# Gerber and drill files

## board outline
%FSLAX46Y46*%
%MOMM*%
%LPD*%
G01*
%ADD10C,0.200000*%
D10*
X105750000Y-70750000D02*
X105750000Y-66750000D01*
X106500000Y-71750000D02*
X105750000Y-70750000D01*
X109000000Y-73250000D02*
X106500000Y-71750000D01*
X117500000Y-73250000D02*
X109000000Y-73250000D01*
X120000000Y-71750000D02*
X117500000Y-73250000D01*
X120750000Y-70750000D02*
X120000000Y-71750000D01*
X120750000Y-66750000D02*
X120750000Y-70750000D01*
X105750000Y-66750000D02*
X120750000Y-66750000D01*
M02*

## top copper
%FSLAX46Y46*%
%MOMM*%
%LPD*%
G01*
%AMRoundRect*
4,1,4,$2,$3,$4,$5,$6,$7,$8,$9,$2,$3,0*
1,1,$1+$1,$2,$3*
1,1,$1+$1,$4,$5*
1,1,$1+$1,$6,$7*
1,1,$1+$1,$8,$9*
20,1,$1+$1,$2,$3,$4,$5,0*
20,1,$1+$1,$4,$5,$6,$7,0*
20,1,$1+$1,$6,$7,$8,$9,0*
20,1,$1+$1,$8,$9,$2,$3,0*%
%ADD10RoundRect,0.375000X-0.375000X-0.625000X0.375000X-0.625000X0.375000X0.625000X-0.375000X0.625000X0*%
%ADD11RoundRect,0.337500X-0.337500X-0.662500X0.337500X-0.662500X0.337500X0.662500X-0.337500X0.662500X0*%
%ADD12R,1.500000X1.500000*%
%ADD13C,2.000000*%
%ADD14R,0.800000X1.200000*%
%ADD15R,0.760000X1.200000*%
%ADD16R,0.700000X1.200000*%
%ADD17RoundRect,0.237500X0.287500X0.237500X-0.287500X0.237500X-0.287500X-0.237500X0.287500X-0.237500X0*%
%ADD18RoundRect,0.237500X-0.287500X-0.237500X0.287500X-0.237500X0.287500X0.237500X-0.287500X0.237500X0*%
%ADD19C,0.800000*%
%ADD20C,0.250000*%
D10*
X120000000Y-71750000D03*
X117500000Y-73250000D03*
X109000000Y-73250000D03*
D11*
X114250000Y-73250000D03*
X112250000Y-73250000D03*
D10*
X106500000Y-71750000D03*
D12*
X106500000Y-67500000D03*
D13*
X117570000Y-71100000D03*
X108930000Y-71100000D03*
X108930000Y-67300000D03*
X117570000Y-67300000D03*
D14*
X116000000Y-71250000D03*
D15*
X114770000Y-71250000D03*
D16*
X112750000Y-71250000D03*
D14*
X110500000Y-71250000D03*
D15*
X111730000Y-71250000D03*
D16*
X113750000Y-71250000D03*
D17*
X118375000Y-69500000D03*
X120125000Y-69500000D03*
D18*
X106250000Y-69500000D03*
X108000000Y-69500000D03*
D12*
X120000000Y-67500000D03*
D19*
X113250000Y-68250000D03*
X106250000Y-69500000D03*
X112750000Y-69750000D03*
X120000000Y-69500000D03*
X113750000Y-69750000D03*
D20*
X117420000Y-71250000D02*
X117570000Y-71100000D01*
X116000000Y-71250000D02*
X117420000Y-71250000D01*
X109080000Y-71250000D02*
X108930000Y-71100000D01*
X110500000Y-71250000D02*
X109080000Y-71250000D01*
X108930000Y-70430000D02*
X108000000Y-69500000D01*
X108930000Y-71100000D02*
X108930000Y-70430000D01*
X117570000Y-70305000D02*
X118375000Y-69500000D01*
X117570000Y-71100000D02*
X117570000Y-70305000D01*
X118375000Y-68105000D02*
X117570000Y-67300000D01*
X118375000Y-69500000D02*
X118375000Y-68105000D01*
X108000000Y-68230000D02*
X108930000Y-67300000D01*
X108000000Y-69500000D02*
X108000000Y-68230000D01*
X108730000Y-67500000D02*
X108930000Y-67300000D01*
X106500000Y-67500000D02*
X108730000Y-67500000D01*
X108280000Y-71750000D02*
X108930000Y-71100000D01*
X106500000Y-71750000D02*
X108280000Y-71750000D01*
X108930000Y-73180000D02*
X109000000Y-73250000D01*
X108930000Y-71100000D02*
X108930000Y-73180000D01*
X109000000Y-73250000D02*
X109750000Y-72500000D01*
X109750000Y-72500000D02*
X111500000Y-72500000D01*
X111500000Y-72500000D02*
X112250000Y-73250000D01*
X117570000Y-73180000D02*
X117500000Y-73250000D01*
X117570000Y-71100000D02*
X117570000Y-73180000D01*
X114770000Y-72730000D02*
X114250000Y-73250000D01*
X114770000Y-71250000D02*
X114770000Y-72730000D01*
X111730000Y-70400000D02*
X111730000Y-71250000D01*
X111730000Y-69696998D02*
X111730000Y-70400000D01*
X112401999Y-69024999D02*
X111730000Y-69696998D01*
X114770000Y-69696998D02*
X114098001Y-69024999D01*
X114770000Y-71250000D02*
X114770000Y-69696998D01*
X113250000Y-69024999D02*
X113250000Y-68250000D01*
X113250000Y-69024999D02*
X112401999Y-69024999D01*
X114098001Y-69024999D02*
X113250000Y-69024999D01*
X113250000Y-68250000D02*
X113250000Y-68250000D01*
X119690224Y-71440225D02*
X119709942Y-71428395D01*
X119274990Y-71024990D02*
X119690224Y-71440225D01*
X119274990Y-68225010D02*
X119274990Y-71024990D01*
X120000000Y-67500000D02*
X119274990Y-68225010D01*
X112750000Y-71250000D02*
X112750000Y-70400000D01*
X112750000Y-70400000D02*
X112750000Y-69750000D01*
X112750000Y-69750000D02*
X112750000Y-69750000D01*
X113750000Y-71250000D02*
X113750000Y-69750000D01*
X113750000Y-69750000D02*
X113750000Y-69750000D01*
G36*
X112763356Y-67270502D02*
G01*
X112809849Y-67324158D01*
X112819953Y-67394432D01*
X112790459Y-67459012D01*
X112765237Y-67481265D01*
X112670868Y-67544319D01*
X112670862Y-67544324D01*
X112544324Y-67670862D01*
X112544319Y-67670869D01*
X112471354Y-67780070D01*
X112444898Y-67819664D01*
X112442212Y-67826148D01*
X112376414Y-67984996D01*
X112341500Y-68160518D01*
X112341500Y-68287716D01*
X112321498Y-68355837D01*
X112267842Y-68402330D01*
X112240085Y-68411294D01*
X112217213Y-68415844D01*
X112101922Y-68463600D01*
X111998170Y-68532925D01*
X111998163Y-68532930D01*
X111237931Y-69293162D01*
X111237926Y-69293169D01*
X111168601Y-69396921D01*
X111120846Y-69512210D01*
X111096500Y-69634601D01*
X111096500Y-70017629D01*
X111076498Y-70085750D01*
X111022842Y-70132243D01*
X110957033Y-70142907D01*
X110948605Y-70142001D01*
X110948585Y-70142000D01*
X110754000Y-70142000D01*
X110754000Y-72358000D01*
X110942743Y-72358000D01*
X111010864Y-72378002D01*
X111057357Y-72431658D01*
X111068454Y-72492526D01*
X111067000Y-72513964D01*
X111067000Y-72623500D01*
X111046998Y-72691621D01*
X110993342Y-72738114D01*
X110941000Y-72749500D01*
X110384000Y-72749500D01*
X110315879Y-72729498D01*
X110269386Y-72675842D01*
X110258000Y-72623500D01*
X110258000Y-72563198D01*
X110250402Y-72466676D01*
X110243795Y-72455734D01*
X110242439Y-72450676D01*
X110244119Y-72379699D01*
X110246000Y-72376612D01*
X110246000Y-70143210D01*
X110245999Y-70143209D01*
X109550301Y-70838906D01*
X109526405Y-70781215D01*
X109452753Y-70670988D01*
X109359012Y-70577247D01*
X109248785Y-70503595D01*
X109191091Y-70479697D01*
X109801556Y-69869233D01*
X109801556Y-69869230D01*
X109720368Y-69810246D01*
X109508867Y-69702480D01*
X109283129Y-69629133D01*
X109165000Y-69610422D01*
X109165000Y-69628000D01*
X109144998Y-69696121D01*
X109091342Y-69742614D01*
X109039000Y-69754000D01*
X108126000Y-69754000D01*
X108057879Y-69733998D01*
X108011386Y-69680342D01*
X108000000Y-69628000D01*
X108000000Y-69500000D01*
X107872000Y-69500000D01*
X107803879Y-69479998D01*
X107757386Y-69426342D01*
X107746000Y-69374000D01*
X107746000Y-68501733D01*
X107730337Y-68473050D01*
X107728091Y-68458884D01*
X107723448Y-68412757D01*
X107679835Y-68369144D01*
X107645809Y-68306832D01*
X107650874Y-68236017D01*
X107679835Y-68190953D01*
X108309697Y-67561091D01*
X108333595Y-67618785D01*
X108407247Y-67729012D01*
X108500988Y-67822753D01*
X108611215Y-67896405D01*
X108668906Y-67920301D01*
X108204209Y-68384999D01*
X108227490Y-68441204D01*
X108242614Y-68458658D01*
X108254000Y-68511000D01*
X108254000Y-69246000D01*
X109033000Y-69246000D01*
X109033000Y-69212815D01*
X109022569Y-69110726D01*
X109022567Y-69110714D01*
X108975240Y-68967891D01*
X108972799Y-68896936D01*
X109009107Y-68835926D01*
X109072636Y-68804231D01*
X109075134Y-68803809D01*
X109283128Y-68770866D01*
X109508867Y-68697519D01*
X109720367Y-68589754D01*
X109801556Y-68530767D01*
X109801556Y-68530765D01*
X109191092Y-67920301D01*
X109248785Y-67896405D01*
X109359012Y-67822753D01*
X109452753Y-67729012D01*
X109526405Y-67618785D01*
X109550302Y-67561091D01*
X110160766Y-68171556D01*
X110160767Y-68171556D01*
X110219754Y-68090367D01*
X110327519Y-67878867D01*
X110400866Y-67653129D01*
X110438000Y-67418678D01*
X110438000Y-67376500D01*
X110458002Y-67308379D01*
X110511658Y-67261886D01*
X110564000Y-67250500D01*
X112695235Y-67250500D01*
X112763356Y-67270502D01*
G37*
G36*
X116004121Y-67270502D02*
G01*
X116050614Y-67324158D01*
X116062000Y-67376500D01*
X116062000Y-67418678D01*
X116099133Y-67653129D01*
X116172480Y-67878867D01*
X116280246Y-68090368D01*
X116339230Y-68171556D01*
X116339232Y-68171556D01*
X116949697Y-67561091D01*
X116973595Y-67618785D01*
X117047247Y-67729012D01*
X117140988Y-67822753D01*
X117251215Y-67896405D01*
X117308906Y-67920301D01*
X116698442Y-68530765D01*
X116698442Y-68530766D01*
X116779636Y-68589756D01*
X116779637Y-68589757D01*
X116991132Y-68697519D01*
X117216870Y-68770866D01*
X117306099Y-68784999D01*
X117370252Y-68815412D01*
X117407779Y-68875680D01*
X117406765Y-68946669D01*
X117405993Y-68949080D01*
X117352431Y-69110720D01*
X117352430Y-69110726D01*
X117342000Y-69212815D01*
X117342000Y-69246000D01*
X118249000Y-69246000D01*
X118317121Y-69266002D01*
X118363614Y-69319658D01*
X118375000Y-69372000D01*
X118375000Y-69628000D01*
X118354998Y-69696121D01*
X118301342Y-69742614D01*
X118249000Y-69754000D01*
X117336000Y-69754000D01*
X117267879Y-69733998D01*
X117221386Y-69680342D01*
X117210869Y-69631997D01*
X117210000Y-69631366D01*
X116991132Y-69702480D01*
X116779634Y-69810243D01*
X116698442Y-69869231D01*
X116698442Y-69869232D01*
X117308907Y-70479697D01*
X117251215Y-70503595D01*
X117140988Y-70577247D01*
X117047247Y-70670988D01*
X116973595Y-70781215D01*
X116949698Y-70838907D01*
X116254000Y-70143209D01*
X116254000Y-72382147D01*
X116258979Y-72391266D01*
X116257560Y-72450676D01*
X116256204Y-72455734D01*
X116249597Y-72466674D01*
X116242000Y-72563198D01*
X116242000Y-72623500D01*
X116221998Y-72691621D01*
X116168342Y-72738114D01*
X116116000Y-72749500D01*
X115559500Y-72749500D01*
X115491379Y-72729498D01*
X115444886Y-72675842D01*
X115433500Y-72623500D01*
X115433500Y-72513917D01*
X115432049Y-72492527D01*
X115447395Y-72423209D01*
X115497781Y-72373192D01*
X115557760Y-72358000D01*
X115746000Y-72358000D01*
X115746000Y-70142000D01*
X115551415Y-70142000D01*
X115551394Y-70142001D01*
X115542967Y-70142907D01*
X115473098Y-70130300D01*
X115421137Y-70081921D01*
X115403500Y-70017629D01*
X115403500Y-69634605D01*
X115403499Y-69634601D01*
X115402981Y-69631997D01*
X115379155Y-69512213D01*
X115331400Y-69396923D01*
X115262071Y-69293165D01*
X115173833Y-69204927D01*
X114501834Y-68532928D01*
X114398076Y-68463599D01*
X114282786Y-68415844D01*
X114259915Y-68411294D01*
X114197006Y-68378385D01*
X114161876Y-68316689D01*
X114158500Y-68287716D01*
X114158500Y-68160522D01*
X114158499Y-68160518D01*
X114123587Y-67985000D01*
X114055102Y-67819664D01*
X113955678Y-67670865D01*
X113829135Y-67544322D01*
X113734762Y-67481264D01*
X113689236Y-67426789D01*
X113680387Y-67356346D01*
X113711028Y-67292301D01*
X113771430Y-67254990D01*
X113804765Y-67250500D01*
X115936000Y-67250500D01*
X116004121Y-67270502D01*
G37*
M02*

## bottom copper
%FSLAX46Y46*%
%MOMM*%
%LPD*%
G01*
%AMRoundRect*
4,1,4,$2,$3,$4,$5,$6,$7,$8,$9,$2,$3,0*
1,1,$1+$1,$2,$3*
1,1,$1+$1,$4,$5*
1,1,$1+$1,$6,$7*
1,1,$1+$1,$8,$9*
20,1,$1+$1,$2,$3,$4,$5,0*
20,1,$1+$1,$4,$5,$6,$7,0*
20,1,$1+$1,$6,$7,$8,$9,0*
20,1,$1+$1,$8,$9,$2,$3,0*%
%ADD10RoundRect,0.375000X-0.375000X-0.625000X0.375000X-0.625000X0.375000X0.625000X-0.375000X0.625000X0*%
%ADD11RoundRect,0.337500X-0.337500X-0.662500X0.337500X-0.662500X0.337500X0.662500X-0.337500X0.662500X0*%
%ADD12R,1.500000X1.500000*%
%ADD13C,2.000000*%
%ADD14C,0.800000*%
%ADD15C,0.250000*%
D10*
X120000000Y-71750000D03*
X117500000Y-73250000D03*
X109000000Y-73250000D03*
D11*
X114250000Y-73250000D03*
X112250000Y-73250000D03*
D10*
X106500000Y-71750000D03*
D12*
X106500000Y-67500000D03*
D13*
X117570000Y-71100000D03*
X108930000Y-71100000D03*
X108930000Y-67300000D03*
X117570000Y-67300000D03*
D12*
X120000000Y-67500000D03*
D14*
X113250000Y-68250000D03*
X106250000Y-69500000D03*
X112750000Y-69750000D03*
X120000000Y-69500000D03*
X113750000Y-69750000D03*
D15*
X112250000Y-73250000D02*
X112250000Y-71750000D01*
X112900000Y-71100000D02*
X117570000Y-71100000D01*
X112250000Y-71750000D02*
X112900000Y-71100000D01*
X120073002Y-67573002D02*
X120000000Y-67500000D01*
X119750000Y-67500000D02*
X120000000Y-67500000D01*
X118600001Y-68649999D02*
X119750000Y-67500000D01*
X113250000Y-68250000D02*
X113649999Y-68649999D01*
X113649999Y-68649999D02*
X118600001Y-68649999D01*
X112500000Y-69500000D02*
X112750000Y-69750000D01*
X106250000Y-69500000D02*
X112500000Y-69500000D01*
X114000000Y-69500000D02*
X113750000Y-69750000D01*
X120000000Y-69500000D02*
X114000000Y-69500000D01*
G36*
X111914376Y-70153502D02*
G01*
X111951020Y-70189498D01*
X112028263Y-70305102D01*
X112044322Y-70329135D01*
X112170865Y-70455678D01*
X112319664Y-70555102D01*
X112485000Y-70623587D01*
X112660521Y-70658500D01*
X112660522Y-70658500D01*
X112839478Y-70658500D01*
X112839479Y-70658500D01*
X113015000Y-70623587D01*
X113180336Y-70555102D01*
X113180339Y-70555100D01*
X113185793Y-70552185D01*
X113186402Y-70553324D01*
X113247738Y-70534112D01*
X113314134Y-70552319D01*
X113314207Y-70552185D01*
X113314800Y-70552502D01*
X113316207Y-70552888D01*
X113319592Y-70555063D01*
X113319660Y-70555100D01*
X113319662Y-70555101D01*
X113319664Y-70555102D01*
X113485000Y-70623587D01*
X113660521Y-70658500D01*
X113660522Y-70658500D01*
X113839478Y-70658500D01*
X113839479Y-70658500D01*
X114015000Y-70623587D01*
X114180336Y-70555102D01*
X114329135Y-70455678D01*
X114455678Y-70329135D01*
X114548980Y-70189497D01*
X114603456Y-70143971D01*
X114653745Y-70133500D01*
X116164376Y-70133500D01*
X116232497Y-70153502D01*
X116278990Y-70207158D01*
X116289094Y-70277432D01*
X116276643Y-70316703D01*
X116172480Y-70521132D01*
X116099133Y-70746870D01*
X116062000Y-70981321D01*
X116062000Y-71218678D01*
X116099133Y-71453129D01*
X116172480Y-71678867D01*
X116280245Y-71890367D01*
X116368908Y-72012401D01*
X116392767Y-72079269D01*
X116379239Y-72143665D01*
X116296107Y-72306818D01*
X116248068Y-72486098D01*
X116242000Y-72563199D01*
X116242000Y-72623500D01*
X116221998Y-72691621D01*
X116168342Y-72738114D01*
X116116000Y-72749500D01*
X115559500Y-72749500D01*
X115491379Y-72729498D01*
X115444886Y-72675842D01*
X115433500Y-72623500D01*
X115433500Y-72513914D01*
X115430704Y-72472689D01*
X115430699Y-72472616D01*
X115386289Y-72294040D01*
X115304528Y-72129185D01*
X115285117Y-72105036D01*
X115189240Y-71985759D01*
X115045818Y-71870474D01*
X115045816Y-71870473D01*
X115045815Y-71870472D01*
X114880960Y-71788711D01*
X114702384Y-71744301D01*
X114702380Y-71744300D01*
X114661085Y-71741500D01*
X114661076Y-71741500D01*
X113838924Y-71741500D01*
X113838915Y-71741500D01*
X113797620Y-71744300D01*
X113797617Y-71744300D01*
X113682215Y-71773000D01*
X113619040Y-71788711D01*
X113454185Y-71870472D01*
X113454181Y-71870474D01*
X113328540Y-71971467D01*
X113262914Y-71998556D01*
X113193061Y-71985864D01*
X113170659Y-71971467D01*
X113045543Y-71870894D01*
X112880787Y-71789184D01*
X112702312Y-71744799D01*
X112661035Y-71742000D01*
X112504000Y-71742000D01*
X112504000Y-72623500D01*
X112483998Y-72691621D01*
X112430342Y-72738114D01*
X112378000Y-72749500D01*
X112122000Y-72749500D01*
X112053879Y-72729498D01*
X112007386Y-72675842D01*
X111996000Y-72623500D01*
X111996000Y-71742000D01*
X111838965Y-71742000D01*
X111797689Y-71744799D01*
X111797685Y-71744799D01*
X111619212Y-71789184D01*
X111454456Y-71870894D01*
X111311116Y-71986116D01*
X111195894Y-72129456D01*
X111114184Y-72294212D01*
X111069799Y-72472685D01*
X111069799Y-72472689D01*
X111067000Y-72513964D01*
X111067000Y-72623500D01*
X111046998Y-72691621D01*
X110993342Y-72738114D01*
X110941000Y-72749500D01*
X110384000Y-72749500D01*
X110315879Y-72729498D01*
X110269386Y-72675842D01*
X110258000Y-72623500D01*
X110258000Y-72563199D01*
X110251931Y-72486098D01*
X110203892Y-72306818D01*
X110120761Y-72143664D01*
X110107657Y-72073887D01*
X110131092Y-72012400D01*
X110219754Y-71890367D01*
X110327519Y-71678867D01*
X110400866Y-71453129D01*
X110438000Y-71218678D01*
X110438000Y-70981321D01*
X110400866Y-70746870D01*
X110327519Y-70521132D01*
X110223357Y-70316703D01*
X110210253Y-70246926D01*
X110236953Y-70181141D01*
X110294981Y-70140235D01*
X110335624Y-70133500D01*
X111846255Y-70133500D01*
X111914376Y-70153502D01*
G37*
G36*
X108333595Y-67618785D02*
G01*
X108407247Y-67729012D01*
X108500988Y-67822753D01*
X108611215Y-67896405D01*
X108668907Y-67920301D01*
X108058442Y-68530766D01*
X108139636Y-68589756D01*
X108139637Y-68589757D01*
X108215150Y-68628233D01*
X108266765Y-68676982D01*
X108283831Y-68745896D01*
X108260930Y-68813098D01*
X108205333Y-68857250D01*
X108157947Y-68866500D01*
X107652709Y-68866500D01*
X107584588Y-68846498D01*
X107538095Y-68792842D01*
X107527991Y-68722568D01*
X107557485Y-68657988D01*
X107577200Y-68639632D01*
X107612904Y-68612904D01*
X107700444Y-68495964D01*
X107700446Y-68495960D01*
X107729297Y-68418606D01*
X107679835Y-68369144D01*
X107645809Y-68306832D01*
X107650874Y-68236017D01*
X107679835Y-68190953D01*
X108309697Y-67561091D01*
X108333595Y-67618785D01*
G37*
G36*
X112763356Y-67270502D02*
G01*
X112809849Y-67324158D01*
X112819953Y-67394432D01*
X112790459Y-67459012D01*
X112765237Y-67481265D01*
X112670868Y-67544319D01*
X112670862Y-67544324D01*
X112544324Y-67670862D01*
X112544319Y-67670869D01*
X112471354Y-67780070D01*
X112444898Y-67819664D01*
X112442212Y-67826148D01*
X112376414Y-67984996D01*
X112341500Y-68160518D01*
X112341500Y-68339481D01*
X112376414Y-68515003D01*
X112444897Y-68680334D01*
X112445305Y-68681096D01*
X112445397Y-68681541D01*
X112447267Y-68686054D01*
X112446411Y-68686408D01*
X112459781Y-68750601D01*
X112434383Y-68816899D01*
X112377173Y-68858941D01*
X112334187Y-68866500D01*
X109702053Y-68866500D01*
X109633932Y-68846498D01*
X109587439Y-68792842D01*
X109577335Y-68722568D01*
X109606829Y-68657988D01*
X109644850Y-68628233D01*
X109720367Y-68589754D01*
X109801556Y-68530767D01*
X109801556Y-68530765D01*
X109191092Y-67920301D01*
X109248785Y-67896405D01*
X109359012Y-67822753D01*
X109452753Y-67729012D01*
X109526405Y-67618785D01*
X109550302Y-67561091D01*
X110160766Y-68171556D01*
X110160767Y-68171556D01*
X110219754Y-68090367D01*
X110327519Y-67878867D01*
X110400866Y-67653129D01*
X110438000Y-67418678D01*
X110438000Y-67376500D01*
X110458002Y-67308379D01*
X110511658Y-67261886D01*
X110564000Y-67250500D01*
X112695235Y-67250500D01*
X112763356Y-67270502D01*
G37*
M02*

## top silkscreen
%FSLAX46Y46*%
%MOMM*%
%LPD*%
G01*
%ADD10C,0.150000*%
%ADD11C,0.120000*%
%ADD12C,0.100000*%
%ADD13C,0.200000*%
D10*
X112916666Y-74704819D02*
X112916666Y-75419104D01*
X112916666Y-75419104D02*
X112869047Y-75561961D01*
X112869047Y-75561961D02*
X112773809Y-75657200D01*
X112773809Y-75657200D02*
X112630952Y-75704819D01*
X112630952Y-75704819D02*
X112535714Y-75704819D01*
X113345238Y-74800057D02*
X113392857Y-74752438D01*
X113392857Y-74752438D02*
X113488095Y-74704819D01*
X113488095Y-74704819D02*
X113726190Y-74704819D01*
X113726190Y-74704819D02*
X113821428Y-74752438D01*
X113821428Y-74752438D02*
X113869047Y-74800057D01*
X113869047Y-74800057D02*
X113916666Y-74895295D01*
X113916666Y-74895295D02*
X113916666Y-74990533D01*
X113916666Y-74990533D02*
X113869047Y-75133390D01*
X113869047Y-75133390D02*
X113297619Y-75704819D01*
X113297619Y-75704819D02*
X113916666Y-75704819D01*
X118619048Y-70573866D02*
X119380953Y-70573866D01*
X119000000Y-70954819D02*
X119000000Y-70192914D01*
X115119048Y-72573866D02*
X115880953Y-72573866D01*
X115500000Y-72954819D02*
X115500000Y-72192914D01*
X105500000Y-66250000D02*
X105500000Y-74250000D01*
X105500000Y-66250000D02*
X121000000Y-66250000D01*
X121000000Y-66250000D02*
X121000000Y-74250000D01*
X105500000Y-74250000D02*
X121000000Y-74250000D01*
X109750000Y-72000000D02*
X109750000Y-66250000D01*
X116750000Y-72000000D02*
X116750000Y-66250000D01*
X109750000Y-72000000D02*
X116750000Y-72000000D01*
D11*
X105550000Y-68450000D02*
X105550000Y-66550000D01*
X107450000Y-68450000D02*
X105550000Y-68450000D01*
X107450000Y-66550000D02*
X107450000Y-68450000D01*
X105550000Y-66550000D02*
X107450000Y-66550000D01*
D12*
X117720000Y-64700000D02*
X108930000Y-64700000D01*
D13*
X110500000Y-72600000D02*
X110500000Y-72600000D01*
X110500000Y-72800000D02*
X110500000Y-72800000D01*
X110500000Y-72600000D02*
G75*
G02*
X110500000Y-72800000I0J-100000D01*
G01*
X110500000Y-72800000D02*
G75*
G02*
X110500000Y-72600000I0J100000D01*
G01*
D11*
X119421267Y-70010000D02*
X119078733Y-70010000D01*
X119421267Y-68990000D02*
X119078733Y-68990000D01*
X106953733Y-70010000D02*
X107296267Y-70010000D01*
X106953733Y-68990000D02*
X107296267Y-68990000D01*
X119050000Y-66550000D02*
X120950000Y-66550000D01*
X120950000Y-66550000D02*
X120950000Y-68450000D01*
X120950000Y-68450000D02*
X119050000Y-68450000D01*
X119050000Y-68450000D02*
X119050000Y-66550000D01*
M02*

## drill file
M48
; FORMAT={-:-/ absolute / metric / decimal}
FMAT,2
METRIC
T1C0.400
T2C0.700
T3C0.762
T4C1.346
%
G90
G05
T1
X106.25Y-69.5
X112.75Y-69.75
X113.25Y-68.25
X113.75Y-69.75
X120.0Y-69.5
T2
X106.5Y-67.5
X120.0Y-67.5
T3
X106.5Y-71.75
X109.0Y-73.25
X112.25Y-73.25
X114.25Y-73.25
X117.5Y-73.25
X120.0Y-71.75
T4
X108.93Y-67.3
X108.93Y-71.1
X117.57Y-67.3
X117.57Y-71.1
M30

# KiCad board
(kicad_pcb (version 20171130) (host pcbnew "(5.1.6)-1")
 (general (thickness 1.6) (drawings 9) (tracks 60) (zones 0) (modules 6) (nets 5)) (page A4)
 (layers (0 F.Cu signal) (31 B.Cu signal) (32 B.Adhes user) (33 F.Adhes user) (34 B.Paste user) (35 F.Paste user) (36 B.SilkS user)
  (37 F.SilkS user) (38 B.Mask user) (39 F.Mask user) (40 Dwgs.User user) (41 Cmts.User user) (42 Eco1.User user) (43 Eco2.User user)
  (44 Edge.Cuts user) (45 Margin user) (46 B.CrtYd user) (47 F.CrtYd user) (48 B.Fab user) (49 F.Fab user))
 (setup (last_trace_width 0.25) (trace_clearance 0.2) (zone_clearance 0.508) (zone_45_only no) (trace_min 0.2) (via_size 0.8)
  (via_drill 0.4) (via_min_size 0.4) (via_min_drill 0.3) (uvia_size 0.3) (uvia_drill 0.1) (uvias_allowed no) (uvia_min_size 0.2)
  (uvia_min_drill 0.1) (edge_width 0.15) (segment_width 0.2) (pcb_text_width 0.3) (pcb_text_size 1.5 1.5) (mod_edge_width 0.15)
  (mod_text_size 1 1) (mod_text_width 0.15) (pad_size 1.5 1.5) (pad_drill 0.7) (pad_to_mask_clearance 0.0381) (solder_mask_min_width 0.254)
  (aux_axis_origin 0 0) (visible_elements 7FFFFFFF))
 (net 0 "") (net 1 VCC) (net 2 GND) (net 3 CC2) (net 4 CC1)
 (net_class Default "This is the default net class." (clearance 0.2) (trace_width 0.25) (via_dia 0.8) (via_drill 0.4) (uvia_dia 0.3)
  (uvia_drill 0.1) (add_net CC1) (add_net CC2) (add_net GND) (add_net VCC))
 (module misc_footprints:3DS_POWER (layer F.Cu) (at 113.25 70.25)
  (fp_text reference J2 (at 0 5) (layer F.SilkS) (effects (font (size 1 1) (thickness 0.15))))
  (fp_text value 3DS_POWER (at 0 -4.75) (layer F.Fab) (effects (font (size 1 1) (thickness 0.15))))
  (fp_line (start -7.75 -4) (end -7.75 4) (layer F.SilkS) (width 0.15))
  (fp_line (start -7.75 -4) (end 7.75 -4) (layer F.SilkS) (width 0.15))
  (fp_line (start 7.75 -4) (end 7.75 4) (layer F.SilkS) (width 0.15))
  (fp_line (start -7.75 4) (end 7.75 4) (layer F.SilkS) (width 0.15))
  (fp_line (start -3.5 1.75) (end -3.5 -4) (layer F.SilkS) (width 0.15))
  (fp_line (start 3.5 1.75) (end 3.5 -4) (layer F.SilkS) (width 0.15))
  (fp_line (start -3.5 1.75) (end 3.5 1.75) (layer F.SilkS) (width 0.15))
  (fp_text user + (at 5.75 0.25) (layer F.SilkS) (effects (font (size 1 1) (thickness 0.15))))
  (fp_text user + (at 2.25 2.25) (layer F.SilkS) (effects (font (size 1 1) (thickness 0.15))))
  (pad 1 thru_hole roundrect (at 6.75 1.5) (size 1.5 2) (drill 0.762) (layers *.Cu *.Mask) (roundrect_rratio 0.25) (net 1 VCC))
  (pad 2 thru_hole roundrect (at 4.25 3) (size 1.5 2) (drill 0.762) (layers *.Cu *.Mask) (roundrect_rratio 0.25) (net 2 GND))
  (pad 2 thru_hole roundrect (at -4.25 3) (size 1.5 2) (drill 0.762) (layers *.Cu *.Mask) (roundrect_rratio 0.25) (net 2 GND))
  (pad 1 thru_hole roundrect (at 1 3) (size 1.35 2) (drill 0.762) (layers *.Cu *.Mask) (roundrect_rratio 0.25) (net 1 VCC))
  (pad 2 thru_hole roundrect (at -1 3) (size 1.35 2) (drill 0.762) (layers *.Cu *.Mask) (roundrect_rratio 0.25) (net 2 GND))
  (pad 2 thru_hole roundrect (at -6.75 1.5) (size 1.5 2) (drill 0.762) (layers *.Cu *.Mask) (roundrect_rratio 0.25) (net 2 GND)))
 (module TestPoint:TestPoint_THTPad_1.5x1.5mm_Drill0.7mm (layer F.Cu) (at 106.5 67.5)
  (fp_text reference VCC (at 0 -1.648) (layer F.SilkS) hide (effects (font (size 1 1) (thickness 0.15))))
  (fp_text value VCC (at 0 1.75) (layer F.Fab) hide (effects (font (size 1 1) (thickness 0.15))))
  (fp_line (start -0.95 0.95) (end -0.95 -0.95) (layer F.SilkS) (width 0.12))
  (fp_line (start 0.95 0.95) (end -0.95 0.95) (layer F.SilkS) (width 0.12))
  (fp_line (start 0.95 -0.95) (end 0.95 0.95) (layer F.SilkS) (width 0.12))
  (fp_line (start -0.95 -0.95) (end 0.95 -0.95) (layer F.SilkS) (width 0.12))
  (pad 1 thru_hole rect (at 0 0) (size 1.5 1.5) (drill 0.7) (layers *.Cu *.Mask) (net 2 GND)))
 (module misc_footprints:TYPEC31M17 (layer F.Cu) (at 113.25 68.75 180)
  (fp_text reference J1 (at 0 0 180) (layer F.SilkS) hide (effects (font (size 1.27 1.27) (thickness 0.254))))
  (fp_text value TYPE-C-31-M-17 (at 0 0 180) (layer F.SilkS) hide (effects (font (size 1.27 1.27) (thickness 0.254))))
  (fp_line (start -4.47 4.05) (end 4.32 4.05) (layer F.SilkS) (width 0.1))
  (fp_line (start 2.75 -3.85) (end 2.75 -3.85) (layer F.SilkS) (width 0.2))
  (fp_line (start 2.75 -4.05) (end 2.75 -4.05) (layer F.SilkS) (width 0.2))
  (fp_arc (start 2.75 -3.95) (end 2.75 -4.05) (angle -180) (layer F.SilkS) (width 0.2))
  (fp_arc (start 2.75 -3.95) (end 2.75 -3.85) (angle -180) (layer F.SilkS) (width 0.2))
  (pad MH4 thru_hole circle (at -4.32 -2.35 180) (size 2 2) (drill 1.346) (layers *.Cu *.Mask) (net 2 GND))
  (pad MH3 thru_hole circle (at 4.32 -2.35 180) (size 2 2) (drill 1.346) (layers *.Cu *.Mask) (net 2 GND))
  (pad MH2 thru_hole circle (at 4.32 1.45 180) (size 2 2) (drill 1.346) (layers *.Cu *.Mask) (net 2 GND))
  (pad MH1 thru_hole circle (at -4.32 1.45 180) (size 2 2) (drill 1.346) (layers *.Cu *.Mask) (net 2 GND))
  (pad B12 smd rect (at -2.75 -2.5 180) (size 0.8 1.2) (layers F.Cu F.Paste F.Mask) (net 2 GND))
  (pad B9 smd rect (at -1.52 -2.5 180) (size 0.76 1.2) (layers F.Cu F.Paste F.Mask) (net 1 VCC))
  (pad B5 smd rect (at 0.5 -2.5 180) (size 0.7 1.2) (layers F.Cu F.Paste F.Mask) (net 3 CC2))
  (pad A12 smd rect (at 2.75 -2.5 180) (size 0.8 1.2) (layers F.Cu F.Paste F.Mask) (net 2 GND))
  (pad A9 smd rect (at 1.52 -2.5 180) (size 0.76 1.2) (layers F.Cu F.Paste F.Mask) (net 1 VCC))
  (pad A5 smd rect (at -0.5 -2.5 180) (size 0.7 1.2) (layers F.Cu F.Paste F.Mask) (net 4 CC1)))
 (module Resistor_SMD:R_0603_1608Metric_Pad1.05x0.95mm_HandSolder (layer F.Cu) (at 119.25 69.5 180)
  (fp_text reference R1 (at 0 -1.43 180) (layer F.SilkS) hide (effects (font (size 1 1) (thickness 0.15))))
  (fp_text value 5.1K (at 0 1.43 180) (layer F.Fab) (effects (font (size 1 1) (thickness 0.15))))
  (fp_line (start -0.171267 -0.51) (end 0.171267 -0.51) (layer F.SilkS) (width 0.12))
  (fp_line (start -0.171267 0.51) (end 0.171267 0.51) (layer F.SilkS) (width 0.12))
  (pad 2 smd roundrect (at 0.875 0 180) (size 1.05 0.95) (layers F.Cu F.Paste F.Mask) (roundrect_rratio 0.25) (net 2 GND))
  (pad 1 smd roundrect (at -0.875 0 180) (size 1.05 0.95) (layers F.Cu F.Paste F.Mask) (roundrect_rratio 0.25) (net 4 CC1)))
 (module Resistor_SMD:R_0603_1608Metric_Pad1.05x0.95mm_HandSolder (layer F.Cu) (at 107.125 69.5)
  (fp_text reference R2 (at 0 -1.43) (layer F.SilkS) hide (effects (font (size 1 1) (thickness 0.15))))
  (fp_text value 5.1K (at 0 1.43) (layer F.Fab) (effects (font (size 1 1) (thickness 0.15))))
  (fp_line (start -0.171267 0.51) (end 0.171267 0.51) (layer F.SilkS) (width 0.12))
  (fp_line (start -0.171267 -0.51) (end 0.171267 -0.51) (layer F.SilkS) (width 0.12))
  (pad 1 smd roundrect (at -0.875 0) (size 1.05 0.95) (layers F.Cu F.Paste F.Mask) (roundrect_rratio 0.25) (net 3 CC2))
  (pad 2 smd roundrect (at 0.875 0) (size 1.05 0.95) (layers F.Cu F.Paste F.Mask) (roundrect_rratio 0.25) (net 2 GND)))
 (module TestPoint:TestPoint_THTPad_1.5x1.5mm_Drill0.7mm (layer F.Cu) (at 120 67.5)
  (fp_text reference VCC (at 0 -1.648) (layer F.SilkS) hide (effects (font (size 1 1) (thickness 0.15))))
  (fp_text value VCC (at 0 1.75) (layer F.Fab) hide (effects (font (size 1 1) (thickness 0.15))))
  (fp_line (start -0.95 -0.95) (end 0.95 -0.95) (layer F.SilkS) (width 0.12))
  (fp_line (start 0.95 -0.95) (end 0.95 0.95) (layer F.SilkS) (width 0.12))
  (fp_line (start 0.95 0.95) (end -0.95 0.95) (layer F.SilkS) (width 0.12))
  (fp_line (start -0.95 0.95) (end -0.95 -0.95) (layer F.SilkS) (width 0.12))
  (pad 1 thru_hole rect (at 0 0) (size 1.5 1.5) (drill 0.7) (layers *.Cu *.Mask) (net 1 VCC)))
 (gr_line (start 105.75 70.75) (end 105.75 66.75) (layer Edge.Cuts) (width 0.2))
 (gr_line (start 106.5 71.75) (end 105.75 70.75) (layer Edge.Cuts) (width 0.2))
 (gr_line (start 109 73.25) (end 106.5 71.75) (layer Edge.Cuts) (width 0.2))
 (gr_line (start 117.5 73.25) (end 109 73.25) (layer Edge.Cuts) (width 0.2))
 (gr_line (start 120 71.75) (end 117.5 73.25) (layer Edge.Cuts) (width 0.2))
 (gr_line (start 120.75 70.75) (end 120 71.75) (layer Edge.Cuts) (width 0.2))
 (gr_line (start 120.75 66.75) (end 120.75 70.75) (layer Edge.Cuts) (width 0.2))
 (gr_line (start 105.75 66.75) (end 120.75 66.75) (layer Edge.Cuts) (width 0.2))
 (segment (start 117.42 71.25) (end 117.57 71.1) (width 0.25) (layer F.Cu) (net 2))
 (segment (start 116 71.25) (end 117.42 71.25) (width 0.25) (layer F.Cu) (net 2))
 (segment (start 109.08 71.25) (end 108.93 71.1) (width 0.25) (layer F.Cu) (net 2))
 (segment (start 110.5 71.25) (end 109.08 71.25) (width 0.25) (layer F.Cu) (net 2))
 (segment (start 108.93 70.43) (end 108 69.5) (width 0.25) (layer F.Cu) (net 2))
 (segment (start 108.93 71.1) (end 108.93 70.43) (width 0.25) (layer F.Cu) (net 2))
 (segment (start 117.57 70.305) (end 118.375 69.5) (width 0.25) (layer F.Cu) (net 2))
 (segment (start 117.57 71.1) (end 117.57 70.305) (width 0.25) (layer F.Cu) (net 2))
 (segment (start 118.375 68.105) (end 117.57 67.3) (width 0.25) (layer F.Cu) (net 2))
 (segment (start 118.375 69.5) (end 118.375 68.105) (width 0.25) (layer F.Cu) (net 2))
 (segment (start 108 68.23) (end 108.93 67.3) (width 0.25) (layer F.Cu) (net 2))
 (segment (start 108 69.5) (end 108 68.23) (width 0.25) (layer F.Cu) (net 2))
 (segment (start 108.73 67.5) (end 108.93 67.3) (width 0.25) (layer F.Cu) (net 2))
 (segment (start 106.5 67.5) (end 108.73 67.5) (width 0.25) (layer F.Cu) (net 2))
 (segment (start 108.28 71.75) (end 108.93 71.1) (width 0.25) (layer F.Cu) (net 2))
 (segment (start 106.5 71.75) (end 108.28 71.75) (width 0.25) (layer F.Cu) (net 2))
 (segment (start 108.93 73.18) (end 109 73.25) (width 0.25) (layer F.Cu) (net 2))
 (segment (start 108.93 71.1) (end 108.93 73.18) (width 0.25) (layer F.Cu) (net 2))
 (segment (start 109 73.25) (end 109.75 72.5) (width 0.25) (layer F.Cu) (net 2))
 (segment (start 109.75 72.5) (end 111.5 72.5) (width 0.25) (layer F.Cu) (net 2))
 (segment (start 111.5 72.5) (end 112.25 73.25) (width 0.25) (layer F.Cu) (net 2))
 (segment (start 117.57 73.18) (end 117.5 73.25) (width 0.25) (layer F.Cu) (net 2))
 (segment (start 117.57 71.1) (end 117.57 73.18) (width 0.25) (layer F.Cu) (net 2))
 (segment (start 112.25 73.25) (end 112.25 71.75) (width 0.25) (layer B.Cu) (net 2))
 (segment (start 112.9 71.1) (end 117.57 71.1) (width 0.25) (layer B.Cu) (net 2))
 (segment (start 112.25 71.75) (end 112.9 71.1) (width 0.25) (layer B.Cu) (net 2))
 (segment (start 114.77 72.73) (end 114.25 73.25) (width 0.25) (layer F.Cu) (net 1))
 (segment (start 114.77 71.25) (end 114.77 72.73) (width 0.25) (layer F.Cu) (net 1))
 (segment (start 111.73 70.4) (end 111.73 71.25) (width 0.25) (layer F.Cu) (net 1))
 (segment (start 111.73 69.696998) (end 111.73 70.4) (width 0.25) (layer F.Cu) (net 1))
 (segment (start 112.401999 69.024999) (end 111.73 69.696998) (width 0.25) (layer F.Cu) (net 1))
 (segment (start 114.77 69.696998) (end 114.098001 69.024999) (width 0.25) (layer F.Cu) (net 1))
 (segment (start 114.77 71.25) (end 114.77 69.696998) (width 0.25) (layer F.Cu) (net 1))
 (segment (start 120.073002 67.573002) (end 120 67.5) (width 0.25) (layer B.Cu) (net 1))
 (segment (start 113.25 69.024999) (end 113.25 68.25) (width 0.25) (layer F.Cu) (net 1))
 (segment (start 113.25 69.024999) (end 112.401999 69.024999) (width 0.25) (layer F.Cu) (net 1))
 (segment (start 114.098001 69.024999) (end 113.25 69.024999) (width 0.25) (layer F.Cu) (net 1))
 (segment (start 113.25 68.25) (end 113.25 68.25) (width 0.25) (layer F.Cu) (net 1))
 (via (at 113.25 68.25) (size 0.8) (drill 0.4) (layers F.Cu B.Cu) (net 1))
 (segment (start 119.75 67.5) (end 120 67.5) (width 0.25) (layer B.Cu) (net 1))
 (segment (start 118.600001 68.649999) (end 119.75 67.5) (width 0.25) (layer B.Cu) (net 1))
 (segment (start 113.25 68.25) (end 113.649999 68.649999) (width 0.25) (layer B.Cu) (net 1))
 (segment (start 113.649999 68.649999) (end 118.600001 68.649999) (width 0.25) (layer B.Cu) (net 1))
 (segment (start 119.690224 71.440225) (end 119.709942 71.428395) (width 0.25) (layer F.Cu) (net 1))
 (segment (start 119.27499 71.02499) (end 119.690224 71.440225) (width 0.25) (layer F.Cu) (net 1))
 (segment (start 119.27499 68.22501) (end 119.27499 71.02499) (width 0.25) (layer F.Cu) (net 1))
 (segment (start 120 67.5) (end 119.27499 68.22501) (width 0.25) (layer F.Cu) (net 1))
 (via (at 106.25 69.5) (size 0.8) (drill 0.4) (layers F.Cu B.Cu) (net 3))
 (segment (start 112.75 71.25) (end 112.75 70.4) (width 0.25) (layer F.Cu) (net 3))
 (segment (start 112.75 70.4) (end 112.75 69.75) (width 0.25) (layer F.Cu) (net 3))
 (segment (start 112.75 69.75) (end 112.75 69.75) (width 0.25) (layer F.Cu) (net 3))
 (via (at 112.75 69.75) (size 0.8) (drill 0.4) (layers F.Cu B.Cu) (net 3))
 (segment (start 112.5 69.5) (end 112.75 69.75) (width 0.25) (layer B.Cu) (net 3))
 (segment (start 106.25 69.5) (end 112.5 69.5) (width 0.25) (layer B.Cu) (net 3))
 (via (at 120 69.5) (size 0.8) (drill 0.4) (layers F.Cu B.Cu) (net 4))
 (segment (start 113.75 71.25) (end 113.75 69.75) (width 0.25) (layer F.Cu) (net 4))
 (segment (start 113.75 69.75) (end 113.75 69.75) (width 0.25) (layer F.Cu) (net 4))
 (via (at 113.75 69.75) (size 0.8) (drill 0.4) (layers F.Cu B.Cu) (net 4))
 (segment (start 114 69.5) (end 113.75 69.75) (width 0.25) (layer B.Cu) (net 4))
 (segment (start 120 69.5) (end 114 69.5) (width 0.25) (layer B.Cu) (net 4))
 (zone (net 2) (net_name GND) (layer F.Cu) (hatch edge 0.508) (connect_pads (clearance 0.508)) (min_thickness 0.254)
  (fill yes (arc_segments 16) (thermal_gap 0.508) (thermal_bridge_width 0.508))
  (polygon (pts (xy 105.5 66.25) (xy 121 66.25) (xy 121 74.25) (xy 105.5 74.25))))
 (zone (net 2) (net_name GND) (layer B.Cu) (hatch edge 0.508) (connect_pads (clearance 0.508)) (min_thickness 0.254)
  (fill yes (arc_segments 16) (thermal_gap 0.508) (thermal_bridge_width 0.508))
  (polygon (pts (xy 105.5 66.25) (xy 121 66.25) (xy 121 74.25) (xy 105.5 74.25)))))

